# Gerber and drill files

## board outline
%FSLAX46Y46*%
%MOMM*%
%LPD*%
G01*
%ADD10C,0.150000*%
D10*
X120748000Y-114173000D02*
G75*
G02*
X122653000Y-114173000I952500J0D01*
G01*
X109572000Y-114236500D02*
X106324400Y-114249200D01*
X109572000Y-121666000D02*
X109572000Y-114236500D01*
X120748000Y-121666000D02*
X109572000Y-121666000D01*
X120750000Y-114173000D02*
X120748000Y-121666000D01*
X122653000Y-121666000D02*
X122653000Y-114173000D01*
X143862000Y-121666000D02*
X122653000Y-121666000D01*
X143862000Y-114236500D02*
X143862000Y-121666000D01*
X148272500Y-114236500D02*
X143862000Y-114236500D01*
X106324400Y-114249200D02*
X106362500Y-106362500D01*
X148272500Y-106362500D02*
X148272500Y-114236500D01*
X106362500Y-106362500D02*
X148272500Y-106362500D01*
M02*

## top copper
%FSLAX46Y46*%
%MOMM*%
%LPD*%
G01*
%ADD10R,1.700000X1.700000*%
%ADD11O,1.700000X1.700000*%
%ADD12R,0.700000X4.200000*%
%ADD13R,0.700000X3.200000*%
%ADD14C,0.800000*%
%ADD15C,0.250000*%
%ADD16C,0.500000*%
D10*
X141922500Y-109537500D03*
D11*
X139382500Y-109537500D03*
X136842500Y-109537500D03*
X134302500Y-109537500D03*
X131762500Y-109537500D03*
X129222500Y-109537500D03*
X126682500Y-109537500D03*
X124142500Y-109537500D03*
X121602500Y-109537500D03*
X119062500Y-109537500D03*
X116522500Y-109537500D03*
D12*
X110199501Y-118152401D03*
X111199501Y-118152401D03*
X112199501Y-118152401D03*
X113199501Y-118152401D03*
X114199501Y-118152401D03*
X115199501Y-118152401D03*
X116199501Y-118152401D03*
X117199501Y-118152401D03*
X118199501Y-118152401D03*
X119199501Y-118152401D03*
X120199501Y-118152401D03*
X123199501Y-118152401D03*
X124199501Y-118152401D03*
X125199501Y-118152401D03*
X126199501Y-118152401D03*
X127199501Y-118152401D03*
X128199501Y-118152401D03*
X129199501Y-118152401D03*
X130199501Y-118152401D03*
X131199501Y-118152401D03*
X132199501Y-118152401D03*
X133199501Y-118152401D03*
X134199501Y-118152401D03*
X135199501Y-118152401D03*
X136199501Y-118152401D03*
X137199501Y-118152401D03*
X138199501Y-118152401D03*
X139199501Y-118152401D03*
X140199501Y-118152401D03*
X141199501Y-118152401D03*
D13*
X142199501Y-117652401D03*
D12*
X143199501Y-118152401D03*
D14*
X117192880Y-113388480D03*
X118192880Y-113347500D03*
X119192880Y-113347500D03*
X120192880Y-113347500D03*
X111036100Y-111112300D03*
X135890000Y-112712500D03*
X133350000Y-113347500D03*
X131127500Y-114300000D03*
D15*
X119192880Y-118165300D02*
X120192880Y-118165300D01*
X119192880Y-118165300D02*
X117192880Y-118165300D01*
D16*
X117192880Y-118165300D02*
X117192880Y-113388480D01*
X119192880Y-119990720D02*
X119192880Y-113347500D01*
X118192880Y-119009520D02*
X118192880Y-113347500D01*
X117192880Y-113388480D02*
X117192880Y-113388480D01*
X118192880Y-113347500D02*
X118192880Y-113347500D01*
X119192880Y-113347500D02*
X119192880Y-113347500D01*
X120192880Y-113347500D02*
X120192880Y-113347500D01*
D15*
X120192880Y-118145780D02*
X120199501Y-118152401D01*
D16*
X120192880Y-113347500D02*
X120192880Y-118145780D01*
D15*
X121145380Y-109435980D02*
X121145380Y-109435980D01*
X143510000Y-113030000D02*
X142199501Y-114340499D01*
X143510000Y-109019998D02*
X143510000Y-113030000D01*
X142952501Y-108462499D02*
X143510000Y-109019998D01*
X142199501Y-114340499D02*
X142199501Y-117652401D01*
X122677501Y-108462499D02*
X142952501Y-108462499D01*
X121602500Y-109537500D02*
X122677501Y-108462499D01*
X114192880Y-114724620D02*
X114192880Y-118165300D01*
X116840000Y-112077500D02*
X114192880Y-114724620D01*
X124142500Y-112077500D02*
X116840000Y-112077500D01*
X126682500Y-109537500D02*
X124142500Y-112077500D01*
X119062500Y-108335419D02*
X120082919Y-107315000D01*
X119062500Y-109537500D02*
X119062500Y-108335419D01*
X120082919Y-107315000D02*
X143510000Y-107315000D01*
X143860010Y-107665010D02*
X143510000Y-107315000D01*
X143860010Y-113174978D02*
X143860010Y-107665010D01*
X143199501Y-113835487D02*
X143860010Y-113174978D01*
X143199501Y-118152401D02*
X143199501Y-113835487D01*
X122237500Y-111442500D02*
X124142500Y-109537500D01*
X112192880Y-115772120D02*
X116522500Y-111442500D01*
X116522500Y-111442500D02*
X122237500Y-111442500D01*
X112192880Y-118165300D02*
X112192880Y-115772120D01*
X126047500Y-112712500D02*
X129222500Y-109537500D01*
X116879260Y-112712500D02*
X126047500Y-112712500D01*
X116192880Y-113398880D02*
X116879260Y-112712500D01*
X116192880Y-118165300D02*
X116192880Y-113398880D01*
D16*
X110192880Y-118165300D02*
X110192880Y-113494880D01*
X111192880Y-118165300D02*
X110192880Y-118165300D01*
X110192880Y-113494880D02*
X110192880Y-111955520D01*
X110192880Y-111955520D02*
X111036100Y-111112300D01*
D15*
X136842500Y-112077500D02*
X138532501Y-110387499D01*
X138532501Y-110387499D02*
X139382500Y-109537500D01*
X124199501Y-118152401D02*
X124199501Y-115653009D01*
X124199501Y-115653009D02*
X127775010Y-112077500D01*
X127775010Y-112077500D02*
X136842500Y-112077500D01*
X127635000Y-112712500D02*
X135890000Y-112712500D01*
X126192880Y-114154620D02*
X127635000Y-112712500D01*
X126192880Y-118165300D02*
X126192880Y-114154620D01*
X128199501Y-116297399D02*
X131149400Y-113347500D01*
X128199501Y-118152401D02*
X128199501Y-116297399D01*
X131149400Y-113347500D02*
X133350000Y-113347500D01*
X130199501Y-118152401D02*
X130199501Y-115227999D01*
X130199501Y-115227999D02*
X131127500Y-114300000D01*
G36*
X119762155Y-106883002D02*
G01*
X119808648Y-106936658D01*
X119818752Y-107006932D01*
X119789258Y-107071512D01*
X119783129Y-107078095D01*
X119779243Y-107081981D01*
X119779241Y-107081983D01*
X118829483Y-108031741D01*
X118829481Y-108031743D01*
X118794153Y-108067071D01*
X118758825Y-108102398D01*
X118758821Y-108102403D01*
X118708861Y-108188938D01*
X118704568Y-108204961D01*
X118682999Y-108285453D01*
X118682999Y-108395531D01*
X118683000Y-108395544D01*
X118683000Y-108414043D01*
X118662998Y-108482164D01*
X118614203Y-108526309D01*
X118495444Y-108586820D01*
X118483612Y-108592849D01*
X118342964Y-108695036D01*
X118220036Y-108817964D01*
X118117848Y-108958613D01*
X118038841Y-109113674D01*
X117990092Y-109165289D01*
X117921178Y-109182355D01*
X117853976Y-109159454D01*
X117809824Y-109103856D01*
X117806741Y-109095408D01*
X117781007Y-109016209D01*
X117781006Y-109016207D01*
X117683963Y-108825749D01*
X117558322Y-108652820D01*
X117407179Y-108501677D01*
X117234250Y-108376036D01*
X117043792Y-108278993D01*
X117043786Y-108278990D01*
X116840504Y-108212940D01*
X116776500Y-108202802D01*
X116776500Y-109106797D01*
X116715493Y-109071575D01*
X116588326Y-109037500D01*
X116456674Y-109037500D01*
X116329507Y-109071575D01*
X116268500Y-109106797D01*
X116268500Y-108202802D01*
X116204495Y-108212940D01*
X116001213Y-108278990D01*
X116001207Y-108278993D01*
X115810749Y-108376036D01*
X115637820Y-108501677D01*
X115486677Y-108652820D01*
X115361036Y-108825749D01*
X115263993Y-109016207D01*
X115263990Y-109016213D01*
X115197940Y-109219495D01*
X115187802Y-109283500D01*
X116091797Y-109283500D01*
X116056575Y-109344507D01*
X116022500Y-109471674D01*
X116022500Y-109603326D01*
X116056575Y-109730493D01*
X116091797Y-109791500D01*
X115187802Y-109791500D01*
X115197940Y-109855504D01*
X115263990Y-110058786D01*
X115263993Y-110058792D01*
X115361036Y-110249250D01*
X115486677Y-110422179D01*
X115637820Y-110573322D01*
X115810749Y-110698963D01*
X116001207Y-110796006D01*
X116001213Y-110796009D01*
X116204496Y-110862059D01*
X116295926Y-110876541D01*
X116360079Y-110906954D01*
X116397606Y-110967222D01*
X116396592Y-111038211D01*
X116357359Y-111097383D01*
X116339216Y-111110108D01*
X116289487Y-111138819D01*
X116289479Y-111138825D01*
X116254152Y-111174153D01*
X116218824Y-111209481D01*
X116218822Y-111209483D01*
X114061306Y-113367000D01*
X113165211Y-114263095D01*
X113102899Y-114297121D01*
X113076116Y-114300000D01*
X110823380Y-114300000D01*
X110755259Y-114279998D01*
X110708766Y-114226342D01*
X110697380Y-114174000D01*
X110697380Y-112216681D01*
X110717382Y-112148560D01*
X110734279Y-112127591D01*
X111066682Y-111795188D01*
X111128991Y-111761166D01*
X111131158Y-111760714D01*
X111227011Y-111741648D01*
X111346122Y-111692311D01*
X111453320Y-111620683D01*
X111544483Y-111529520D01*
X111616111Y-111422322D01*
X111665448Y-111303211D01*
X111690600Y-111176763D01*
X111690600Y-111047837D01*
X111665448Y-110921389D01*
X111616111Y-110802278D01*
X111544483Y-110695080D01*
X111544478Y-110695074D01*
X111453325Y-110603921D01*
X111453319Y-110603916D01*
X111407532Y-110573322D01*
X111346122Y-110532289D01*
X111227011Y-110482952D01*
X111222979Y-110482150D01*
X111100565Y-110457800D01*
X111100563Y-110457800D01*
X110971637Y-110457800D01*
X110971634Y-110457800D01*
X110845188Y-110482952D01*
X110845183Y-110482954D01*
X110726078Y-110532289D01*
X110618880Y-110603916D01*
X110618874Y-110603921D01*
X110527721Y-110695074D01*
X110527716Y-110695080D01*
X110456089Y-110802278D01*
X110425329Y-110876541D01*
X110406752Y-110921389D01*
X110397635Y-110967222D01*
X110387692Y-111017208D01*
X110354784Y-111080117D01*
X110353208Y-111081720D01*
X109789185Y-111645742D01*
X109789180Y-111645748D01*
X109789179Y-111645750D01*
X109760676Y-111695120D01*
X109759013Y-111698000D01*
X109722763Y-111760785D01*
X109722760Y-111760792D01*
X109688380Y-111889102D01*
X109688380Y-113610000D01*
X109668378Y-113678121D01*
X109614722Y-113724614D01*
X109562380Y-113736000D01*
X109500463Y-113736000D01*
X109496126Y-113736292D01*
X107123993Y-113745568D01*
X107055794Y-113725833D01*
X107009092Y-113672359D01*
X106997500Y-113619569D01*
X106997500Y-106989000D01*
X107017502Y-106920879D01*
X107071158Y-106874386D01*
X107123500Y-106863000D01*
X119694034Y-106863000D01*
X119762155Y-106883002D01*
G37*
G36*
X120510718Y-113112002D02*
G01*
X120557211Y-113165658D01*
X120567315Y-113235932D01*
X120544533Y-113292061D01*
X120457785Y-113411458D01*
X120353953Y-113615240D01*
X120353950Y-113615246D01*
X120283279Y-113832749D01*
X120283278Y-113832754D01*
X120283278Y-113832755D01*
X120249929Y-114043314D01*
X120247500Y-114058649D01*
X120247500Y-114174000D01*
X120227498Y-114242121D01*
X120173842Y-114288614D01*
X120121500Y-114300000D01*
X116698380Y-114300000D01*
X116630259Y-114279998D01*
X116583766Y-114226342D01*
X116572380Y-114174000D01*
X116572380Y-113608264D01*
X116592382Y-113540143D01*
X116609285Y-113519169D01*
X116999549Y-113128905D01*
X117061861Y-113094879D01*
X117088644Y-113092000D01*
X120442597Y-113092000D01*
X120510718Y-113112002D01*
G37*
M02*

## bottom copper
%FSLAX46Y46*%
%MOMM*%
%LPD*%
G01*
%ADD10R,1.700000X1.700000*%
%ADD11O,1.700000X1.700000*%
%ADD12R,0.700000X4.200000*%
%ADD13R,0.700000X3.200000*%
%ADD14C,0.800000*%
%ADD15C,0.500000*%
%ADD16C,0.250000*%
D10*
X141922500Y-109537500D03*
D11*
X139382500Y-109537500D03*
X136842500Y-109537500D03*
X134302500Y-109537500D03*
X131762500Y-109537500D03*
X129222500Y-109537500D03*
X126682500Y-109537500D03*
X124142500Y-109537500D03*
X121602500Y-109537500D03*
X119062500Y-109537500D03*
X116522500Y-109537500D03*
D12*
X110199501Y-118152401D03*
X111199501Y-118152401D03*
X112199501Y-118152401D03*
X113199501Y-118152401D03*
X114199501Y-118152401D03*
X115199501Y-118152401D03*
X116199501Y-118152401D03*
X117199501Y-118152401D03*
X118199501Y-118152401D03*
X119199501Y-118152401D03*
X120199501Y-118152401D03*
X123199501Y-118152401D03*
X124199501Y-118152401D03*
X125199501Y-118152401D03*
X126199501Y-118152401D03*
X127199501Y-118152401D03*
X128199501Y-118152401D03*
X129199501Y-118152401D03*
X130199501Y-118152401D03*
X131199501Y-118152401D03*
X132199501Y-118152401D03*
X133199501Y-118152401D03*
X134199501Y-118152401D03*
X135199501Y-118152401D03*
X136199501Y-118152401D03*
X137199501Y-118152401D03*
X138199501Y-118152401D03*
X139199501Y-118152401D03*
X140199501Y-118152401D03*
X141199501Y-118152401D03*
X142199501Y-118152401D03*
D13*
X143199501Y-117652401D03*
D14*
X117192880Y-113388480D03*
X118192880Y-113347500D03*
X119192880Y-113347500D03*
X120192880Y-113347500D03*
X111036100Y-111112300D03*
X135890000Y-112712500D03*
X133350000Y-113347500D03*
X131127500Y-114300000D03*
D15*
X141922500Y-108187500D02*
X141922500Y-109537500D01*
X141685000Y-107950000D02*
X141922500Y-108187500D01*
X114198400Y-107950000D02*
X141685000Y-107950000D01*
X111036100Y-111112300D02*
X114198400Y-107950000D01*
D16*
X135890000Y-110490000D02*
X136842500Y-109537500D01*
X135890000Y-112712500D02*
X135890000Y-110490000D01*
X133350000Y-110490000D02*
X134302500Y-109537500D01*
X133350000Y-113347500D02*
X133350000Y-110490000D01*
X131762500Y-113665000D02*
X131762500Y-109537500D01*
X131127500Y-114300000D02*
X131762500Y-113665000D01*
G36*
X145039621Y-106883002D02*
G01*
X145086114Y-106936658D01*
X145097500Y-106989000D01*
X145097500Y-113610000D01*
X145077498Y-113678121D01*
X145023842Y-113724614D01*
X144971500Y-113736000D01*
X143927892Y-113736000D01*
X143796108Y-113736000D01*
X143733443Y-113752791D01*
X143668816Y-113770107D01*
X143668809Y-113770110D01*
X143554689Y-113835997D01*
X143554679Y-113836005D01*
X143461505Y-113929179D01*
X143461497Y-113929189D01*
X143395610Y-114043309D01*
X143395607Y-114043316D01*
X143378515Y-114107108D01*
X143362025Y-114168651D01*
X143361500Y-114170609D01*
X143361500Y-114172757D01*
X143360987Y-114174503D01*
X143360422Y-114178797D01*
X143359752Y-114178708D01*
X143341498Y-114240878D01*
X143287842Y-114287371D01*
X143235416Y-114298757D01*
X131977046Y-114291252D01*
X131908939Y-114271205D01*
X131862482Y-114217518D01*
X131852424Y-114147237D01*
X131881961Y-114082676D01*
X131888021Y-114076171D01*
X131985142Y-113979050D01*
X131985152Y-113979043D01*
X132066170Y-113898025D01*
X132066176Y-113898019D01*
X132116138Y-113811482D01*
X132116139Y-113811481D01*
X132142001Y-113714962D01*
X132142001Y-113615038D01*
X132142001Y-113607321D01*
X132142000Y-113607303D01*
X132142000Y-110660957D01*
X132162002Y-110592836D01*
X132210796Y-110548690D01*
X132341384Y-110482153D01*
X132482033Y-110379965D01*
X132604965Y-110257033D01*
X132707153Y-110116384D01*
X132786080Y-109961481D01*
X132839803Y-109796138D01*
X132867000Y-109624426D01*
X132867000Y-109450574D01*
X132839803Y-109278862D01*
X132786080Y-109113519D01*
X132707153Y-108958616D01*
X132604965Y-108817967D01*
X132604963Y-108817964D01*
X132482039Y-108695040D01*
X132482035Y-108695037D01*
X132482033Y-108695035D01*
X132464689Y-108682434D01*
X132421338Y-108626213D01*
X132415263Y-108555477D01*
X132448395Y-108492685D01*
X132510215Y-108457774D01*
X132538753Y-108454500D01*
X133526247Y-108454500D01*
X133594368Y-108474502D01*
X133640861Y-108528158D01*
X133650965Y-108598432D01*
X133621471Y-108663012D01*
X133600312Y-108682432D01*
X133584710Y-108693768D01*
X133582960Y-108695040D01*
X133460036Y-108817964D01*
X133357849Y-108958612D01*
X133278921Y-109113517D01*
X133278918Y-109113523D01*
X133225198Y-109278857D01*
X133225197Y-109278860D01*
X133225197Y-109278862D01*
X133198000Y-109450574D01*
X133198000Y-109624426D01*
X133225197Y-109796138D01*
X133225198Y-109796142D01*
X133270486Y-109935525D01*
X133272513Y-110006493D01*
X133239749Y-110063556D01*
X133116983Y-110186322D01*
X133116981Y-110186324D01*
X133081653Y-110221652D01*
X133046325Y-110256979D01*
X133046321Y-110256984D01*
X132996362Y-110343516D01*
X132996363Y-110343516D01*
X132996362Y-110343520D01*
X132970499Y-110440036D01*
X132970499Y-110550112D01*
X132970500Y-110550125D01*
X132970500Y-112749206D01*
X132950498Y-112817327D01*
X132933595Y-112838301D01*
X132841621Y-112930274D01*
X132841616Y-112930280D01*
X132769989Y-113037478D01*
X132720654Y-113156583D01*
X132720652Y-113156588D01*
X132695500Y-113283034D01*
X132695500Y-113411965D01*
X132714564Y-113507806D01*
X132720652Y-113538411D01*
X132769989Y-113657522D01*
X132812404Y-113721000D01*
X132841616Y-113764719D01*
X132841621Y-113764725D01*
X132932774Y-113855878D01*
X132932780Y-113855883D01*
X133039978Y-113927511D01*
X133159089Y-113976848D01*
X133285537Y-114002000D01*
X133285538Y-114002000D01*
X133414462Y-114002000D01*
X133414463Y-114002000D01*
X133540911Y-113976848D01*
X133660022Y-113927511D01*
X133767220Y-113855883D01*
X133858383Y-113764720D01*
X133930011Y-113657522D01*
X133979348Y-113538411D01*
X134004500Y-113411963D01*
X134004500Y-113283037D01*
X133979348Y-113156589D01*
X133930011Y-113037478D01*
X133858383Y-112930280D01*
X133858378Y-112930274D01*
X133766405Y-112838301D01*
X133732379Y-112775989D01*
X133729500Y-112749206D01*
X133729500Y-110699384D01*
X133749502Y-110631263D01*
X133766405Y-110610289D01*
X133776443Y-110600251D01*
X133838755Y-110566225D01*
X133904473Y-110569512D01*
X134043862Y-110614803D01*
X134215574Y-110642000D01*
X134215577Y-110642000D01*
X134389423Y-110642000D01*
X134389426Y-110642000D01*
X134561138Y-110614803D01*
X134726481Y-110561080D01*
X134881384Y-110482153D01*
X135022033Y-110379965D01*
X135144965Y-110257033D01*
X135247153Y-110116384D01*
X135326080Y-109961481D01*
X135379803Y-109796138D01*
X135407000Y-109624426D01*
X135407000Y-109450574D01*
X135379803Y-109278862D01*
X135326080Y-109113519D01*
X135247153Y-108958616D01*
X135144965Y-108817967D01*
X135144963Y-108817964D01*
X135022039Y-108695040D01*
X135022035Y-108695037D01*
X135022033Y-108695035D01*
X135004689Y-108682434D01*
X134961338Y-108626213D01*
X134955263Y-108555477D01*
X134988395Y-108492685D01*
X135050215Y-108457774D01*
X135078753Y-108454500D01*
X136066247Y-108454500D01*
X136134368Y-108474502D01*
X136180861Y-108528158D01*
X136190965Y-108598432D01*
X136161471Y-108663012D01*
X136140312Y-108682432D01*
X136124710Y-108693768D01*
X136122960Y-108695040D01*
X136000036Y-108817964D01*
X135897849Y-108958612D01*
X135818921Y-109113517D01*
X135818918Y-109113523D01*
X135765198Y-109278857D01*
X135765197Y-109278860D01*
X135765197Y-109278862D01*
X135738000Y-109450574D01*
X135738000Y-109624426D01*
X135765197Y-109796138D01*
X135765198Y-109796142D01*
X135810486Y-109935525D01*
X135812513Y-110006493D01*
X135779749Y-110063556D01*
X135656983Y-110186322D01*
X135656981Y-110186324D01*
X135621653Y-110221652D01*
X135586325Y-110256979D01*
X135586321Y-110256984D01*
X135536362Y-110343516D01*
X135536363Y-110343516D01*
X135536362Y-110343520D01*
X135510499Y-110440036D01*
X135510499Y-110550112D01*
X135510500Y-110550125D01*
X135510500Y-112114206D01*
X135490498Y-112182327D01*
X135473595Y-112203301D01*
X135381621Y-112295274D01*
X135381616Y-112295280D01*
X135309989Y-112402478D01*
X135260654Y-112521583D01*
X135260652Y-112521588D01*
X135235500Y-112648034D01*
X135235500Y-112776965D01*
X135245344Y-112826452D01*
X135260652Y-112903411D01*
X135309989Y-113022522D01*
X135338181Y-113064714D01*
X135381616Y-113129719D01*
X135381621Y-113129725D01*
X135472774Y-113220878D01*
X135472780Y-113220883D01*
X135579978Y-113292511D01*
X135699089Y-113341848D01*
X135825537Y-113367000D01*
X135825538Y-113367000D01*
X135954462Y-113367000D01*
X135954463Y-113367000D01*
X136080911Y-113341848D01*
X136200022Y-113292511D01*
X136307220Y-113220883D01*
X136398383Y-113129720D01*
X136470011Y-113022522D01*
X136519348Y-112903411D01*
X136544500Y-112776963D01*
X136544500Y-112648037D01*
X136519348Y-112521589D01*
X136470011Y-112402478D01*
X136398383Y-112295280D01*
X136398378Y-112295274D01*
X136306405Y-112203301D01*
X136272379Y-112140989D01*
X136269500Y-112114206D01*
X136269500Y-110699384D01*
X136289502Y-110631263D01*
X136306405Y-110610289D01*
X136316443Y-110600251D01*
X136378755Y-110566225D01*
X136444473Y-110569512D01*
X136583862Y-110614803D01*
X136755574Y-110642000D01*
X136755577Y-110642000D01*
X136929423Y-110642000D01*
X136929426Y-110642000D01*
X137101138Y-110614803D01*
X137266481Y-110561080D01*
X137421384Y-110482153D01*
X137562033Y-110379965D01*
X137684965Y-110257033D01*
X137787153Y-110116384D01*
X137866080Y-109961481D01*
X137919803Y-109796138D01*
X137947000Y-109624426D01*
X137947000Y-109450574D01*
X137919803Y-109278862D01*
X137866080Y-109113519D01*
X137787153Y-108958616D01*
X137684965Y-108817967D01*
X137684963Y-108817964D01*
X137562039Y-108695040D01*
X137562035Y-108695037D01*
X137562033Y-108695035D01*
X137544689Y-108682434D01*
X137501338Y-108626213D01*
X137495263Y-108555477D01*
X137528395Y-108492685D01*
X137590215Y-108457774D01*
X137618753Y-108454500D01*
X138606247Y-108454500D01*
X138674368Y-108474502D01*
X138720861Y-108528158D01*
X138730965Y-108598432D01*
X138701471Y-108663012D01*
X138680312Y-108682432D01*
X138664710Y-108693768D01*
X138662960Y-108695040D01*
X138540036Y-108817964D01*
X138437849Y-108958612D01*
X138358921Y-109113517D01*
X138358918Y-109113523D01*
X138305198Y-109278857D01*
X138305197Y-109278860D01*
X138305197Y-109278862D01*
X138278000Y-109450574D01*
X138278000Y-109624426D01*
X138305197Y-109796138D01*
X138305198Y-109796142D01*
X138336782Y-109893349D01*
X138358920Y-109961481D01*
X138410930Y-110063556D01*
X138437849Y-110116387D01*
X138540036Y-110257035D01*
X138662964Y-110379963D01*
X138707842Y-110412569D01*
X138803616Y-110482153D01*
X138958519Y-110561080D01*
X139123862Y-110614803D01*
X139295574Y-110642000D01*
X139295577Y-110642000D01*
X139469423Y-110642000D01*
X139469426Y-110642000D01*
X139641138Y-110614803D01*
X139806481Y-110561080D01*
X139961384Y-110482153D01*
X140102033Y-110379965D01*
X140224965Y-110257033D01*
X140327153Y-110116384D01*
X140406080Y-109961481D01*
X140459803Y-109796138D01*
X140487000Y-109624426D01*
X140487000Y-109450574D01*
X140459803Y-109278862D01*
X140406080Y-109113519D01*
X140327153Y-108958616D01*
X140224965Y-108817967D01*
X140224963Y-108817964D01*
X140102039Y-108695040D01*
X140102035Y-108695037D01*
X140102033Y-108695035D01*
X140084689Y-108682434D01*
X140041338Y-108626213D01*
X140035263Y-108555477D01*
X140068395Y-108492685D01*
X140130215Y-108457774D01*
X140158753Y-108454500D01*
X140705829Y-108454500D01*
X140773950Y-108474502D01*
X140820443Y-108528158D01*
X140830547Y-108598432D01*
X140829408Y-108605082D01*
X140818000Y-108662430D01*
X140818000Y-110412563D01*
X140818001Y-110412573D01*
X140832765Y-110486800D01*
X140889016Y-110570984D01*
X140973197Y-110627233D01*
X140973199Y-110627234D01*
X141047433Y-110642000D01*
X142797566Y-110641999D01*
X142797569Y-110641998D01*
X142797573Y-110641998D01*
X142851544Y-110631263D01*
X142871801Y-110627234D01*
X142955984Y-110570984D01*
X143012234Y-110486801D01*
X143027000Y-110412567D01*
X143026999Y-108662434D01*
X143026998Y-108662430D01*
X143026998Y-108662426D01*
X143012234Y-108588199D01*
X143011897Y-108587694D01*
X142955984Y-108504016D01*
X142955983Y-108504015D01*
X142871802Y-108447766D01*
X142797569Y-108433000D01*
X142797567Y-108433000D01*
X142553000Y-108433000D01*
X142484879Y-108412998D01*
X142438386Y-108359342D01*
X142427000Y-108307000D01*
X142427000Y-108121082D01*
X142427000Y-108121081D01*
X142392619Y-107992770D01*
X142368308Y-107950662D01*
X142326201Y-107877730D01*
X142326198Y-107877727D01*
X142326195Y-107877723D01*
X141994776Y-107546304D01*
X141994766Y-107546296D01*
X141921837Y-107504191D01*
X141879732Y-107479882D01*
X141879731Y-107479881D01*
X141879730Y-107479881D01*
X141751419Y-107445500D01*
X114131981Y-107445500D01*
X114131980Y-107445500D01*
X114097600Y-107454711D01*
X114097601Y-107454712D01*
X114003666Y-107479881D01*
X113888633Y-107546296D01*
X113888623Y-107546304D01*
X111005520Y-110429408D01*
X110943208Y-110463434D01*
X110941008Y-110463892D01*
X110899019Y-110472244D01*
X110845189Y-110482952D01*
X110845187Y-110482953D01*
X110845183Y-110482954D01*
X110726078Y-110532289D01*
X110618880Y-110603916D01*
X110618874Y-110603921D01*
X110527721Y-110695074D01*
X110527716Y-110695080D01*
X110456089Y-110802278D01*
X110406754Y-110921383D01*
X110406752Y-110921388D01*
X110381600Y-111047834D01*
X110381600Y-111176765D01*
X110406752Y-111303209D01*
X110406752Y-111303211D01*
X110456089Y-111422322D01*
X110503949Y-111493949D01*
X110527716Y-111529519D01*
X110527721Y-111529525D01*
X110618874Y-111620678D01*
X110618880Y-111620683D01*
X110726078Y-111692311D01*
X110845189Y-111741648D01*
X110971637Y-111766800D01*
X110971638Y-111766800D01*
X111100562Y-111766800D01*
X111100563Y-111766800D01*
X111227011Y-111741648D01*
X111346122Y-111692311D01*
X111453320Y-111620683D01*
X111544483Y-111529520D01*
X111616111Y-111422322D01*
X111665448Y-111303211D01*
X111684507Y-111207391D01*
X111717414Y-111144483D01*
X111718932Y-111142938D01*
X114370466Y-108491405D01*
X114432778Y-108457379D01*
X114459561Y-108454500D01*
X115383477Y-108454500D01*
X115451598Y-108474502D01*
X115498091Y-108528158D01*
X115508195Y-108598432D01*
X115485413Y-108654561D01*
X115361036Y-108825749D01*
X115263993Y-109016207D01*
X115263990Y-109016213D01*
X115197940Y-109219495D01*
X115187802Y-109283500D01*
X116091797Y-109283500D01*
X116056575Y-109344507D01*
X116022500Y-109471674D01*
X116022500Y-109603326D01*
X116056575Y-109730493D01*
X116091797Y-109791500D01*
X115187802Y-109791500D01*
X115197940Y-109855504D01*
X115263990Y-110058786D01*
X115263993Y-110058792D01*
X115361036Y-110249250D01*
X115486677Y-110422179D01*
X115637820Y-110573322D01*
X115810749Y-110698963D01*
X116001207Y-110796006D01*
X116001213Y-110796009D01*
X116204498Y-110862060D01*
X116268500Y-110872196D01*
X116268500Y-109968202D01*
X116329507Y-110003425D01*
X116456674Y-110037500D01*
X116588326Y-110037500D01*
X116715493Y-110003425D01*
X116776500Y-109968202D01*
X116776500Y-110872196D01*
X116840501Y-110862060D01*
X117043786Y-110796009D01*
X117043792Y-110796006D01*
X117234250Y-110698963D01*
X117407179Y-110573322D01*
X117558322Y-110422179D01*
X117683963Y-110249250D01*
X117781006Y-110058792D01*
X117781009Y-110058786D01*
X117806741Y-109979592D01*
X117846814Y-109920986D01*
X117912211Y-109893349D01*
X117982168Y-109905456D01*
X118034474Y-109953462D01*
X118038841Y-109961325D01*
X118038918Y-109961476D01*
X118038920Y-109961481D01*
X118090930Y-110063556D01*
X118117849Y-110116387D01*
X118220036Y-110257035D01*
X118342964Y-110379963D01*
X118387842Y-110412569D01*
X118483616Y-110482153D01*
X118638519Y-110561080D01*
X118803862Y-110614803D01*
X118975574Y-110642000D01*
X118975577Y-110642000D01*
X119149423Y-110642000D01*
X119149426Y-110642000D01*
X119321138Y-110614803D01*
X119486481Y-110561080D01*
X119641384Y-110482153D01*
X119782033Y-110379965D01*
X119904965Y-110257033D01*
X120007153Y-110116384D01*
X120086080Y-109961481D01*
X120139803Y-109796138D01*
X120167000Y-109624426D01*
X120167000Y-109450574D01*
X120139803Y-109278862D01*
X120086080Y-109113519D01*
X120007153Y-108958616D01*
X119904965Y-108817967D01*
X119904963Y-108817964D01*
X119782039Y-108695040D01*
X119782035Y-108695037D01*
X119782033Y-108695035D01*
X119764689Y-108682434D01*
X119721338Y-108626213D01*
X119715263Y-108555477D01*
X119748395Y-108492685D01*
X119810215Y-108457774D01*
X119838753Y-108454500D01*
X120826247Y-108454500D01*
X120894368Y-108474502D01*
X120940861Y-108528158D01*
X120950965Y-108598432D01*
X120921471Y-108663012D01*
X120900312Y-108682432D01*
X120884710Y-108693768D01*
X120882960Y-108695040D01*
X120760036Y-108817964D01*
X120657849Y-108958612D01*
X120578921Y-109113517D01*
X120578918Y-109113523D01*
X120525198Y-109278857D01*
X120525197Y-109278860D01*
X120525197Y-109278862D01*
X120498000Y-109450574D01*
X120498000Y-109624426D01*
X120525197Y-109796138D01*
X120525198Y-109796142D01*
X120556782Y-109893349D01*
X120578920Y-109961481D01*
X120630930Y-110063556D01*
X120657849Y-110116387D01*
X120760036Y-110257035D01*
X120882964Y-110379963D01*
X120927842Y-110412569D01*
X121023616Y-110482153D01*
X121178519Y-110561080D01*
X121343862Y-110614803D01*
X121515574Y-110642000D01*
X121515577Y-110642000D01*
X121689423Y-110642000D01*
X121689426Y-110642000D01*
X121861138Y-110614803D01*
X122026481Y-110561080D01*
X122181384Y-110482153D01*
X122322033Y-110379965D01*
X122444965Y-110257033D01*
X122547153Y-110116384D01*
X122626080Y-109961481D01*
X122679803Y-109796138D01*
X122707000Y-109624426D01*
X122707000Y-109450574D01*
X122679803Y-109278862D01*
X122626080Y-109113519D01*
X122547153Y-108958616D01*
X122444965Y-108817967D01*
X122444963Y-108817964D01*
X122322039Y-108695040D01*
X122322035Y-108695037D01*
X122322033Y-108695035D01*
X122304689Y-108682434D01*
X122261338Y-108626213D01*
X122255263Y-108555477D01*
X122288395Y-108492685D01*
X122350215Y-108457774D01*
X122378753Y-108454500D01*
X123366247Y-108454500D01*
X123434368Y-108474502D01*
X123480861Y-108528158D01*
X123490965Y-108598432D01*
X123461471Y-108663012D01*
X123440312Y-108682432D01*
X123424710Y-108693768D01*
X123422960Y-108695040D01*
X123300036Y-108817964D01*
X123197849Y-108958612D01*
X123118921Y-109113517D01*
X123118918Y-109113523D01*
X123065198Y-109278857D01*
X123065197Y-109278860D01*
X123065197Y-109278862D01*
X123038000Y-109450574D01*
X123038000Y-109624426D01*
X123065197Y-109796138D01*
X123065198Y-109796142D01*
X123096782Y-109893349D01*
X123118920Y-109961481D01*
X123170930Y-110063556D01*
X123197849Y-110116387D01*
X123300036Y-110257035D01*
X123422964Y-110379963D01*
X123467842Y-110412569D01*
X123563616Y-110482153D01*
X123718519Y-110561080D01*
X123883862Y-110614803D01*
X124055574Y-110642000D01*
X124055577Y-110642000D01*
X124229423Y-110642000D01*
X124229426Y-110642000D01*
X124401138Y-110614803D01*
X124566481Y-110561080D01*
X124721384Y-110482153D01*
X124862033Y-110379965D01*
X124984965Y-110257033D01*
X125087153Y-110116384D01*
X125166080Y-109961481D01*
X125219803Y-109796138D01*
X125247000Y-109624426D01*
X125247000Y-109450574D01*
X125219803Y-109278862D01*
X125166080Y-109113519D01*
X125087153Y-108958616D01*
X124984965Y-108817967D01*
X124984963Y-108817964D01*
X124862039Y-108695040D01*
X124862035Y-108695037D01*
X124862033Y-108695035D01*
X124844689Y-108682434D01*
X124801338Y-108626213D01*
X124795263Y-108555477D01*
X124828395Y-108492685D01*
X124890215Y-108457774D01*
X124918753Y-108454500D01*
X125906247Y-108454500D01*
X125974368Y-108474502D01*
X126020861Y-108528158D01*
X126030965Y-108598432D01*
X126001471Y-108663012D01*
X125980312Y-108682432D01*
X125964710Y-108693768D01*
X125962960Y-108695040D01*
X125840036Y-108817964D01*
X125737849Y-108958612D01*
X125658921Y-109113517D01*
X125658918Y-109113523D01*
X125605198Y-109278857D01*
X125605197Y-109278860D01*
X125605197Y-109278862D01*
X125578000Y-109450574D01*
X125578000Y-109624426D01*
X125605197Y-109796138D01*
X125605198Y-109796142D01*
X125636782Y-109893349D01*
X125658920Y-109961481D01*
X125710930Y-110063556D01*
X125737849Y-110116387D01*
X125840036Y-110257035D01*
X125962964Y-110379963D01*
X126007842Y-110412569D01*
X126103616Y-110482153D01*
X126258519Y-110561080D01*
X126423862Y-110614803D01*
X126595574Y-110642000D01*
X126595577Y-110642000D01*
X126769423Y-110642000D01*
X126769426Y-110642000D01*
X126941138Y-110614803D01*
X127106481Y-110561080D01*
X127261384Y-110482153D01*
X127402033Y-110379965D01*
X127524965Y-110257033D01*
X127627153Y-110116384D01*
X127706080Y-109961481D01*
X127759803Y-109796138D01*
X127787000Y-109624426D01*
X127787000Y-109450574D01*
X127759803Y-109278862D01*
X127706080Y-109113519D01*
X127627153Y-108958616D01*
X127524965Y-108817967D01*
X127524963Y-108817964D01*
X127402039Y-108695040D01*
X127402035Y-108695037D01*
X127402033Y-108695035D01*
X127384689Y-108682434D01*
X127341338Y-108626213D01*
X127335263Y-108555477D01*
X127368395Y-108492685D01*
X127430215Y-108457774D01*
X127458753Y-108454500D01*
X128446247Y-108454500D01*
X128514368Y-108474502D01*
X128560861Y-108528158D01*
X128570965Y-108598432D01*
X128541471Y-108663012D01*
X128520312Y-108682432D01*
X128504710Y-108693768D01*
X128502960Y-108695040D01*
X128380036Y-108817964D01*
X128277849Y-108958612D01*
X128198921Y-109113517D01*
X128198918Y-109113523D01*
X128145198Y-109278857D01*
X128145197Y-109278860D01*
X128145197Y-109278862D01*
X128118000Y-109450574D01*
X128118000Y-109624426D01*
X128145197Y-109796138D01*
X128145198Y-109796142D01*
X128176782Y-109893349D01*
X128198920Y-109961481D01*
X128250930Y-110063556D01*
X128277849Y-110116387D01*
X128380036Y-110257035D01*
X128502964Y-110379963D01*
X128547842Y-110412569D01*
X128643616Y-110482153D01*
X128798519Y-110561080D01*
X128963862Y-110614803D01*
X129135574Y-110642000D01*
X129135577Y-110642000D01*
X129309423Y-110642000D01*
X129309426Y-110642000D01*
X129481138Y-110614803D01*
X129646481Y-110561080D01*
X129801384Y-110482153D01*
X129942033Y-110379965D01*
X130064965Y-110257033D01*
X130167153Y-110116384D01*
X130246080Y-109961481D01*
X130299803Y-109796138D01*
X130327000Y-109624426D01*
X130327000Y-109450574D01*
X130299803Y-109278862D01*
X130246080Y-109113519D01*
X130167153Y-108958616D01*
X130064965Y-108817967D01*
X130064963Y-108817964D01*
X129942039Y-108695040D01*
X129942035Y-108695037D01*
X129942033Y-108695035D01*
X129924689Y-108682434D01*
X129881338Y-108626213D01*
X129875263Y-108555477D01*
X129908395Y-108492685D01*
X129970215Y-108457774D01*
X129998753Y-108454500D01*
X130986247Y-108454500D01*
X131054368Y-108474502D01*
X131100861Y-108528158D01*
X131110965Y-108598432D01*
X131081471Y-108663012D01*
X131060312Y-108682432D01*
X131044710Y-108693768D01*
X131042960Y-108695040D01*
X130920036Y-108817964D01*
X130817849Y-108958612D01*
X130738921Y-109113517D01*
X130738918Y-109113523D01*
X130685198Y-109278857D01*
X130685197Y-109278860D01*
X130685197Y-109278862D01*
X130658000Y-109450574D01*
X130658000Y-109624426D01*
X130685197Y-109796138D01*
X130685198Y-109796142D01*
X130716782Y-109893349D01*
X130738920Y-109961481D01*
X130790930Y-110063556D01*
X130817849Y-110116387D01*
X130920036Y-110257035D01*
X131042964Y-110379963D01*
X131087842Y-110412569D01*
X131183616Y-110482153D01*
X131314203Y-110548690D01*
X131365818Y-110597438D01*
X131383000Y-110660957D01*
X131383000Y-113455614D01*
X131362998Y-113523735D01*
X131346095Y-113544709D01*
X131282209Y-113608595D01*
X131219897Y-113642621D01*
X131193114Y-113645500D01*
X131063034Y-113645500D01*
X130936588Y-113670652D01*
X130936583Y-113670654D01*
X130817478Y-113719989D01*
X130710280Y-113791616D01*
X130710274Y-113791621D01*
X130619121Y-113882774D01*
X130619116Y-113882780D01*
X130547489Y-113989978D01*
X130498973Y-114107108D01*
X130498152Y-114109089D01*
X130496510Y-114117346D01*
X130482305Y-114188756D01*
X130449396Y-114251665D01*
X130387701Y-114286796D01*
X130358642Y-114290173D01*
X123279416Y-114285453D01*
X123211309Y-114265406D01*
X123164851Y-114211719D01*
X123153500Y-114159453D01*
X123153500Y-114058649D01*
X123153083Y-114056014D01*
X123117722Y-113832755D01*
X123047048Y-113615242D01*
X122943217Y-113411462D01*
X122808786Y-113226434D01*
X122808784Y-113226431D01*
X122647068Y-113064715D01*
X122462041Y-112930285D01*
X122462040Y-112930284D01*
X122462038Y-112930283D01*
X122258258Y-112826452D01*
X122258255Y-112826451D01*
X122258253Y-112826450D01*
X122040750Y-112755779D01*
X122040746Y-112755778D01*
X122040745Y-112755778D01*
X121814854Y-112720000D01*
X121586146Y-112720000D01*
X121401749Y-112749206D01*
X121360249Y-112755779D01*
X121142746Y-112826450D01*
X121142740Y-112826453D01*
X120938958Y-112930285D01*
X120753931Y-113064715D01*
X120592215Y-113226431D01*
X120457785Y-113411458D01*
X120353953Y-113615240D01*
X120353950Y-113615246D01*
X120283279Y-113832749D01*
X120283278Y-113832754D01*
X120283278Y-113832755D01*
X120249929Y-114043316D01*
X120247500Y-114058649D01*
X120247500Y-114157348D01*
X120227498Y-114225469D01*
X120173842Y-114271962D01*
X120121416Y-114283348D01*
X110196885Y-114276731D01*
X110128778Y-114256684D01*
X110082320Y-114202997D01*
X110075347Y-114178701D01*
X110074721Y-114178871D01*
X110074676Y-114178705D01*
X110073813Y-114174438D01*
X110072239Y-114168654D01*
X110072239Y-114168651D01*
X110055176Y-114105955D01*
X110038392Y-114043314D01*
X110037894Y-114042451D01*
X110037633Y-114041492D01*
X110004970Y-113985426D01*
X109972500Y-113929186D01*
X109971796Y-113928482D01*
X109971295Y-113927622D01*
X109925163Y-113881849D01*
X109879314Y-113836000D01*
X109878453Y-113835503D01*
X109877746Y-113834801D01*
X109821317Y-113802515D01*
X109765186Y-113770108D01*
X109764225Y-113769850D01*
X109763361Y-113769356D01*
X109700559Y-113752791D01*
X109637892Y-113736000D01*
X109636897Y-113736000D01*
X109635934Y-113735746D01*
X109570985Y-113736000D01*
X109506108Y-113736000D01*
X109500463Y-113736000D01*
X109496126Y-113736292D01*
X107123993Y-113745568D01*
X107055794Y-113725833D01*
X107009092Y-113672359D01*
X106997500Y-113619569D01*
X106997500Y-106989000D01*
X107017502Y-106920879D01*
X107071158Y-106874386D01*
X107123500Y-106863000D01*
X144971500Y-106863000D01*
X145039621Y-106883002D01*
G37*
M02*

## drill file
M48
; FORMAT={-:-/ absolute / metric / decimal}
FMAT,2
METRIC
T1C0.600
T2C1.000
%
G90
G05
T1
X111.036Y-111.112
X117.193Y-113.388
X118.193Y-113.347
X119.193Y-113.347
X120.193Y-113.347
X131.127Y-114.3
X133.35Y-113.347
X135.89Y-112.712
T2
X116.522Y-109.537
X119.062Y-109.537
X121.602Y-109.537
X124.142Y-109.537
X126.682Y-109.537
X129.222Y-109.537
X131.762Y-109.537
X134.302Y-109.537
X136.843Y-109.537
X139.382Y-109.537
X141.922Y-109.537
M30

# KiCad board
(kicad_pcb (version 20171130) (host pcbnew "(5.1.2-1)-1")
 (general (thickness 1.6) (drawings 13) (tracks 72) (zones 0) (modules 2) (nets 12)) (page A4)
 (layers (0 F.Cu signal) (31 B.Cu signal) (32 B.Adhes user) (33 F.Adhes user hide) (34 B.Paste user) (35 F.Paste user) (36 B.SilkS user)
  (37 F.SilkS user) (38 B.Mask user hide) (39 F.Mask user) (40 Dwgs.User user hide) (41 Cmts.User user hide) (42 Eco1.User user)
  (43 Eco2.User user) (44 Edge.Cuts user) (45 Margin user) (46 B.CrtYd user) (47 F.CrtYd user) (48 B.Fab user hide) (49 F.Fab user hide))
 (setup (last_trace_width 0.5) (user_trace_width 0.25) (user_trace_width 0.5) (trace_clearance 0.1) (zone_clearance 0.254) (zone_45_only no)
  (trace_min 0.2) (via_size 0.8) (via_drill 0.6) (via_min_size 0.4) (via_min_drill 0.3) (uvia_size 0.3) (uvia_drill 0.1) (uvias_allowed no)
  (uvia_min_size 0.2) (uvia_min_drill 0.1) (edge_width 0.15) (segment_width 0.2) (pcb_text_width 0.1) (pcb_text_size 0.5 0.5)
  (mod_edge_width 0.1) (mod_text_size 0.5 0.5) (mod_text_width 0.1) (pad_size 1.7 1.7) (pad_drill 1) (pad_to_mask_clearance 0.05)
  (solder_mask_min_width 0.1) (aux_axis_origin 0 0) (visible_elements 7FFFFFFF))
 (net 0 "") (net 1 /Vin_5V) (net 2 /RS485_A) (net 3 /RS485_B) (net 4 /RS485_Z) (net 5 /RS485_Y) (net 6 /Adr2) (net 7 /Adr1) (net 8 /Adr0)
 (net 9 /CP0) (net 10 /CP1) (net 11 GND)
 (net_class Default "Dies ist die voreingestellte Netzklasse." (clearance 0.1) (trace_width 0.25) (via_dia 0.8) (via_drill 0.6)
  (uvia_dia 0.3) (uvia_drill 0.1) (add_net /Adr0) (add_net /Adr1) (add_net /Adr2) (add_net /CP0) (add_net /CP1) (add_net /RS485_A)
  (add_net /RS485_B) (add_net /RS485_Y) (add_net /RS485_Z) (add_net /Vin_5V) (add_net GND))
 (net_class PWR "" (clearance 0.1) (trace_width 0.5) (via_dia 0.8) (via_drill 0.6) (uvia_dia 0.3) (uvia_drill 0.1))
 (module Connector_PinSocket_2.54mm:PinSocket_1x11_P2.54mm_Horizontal (layer F.Cu) (at 141.9225 109.5375 270)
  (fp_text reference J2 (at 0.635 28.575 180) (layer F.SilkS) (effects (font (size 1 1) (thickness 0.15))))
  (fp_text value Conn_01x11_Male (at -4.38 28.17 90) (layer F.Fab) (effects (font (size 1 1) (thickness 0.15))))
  (pad 1 thru_hole rect (at 0 0 270) (size 1.7 1.7) (drill 1) (layers *.Cu *.Mask) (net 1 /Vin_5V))
  (pad 2 thru_hole oval (at 0 2.54 270) (size 1.7 1.7) (drill 1) (layers *.Cu *.Mask) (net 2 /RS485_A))
  (pad 3 thru_hole oval (at 0 5.08 270) (size 1.7 1.7) (drill 1) (layers *.Cu *.Mask) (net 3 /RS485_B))
  (pad 4 thru_hole oval (at 0 7.62 270) (size 1.7 1.7) (drill 1) (layers *.Cu *.Mask) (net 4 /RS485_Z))
  (pad 5 thru_hole oval (at 0 10.16 270) (size 1.7 1.7) (drill 1) (layers *.Cu *.Mask) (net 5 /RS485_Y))
  (pad 6 thru_hole oval (at 0 12.7 270) (size 1.7 1.7) (drill 1) (layers *.Cu *.Mask) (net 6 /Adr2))
  (pad 7 thru_hole oval (at 0 15.24 270) (size 1.7 1.7) (drill 1) (layers *.Cu *.Mask) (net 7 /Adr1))
  (pad 8 thru_hole oval (at 0 17.78 270) (size 1.7 1.7) (drill 1) (layers *.Cu *.Mask) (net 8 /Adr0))
  (pad 9 thru_hole oval (at 0 20.32 270) (size 1.7 1.7) (drill 1) (layers *.Cu *.Mask) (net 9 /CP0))
  (pad 10 thru_hole oval (at 0 22.86 270) (size 1.7 1.7) (drill 1) (layers *.Cu *.Mask) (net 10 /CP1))
  (pad 11 thru_hole oval (at 0 25.4 270) (size 1.7 1.7) (drill 1) (layers *.Cu *.Mask) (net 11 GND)))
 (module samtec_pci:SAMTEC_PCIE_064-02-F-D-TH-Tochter (layer F.Cu) (at 121.699501 116.052401)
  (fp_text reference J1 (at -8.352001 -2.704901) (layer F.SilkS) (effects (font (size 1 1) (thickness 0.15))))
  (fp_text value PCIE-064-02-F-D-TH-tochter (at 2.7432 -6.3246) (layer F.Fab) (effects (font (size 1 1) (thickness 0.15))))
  (pad B1 connect rect (at -11.5 2.1) (size 0.7 4.2) (layers F.Cu F.Mask) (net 1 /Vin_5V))
  (pad B2 connect rect (at -10.5 2.1) (size 0.7 4.2) (layers F.Cu F.Mask) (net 1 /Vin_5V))
  (pad B3 connect rect (at -9.5 2.1) (size 0.7 4.2) (layers F.Cu F.Mask) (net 8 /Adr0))
  (pad B4 connect rect (at -8.5 2.1) (size 0.7 4.2) (layers F.Cu F.Mask))
  (pad B5 connect rect (at -7.5 2.1) (size 0.7 4.2) (layers F.Cu F.Mask) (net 7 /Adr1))
  (pad B6 connect rect (at -6.5 2.1) (size 0.7 4.2) (layers F.Cu F.Mask))
  (pad B7 connect rect (at -5.5 2.1) (size 0.7 4.2) (layers F.Cu F.Mask) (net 6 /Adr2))
  (pad B8 connect rect (at -4.5 2.1) (size 0.7 4.2) (layers F.Cu F.Mask) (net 11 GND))
  (pad B9 connect rect (at -3.5 2.1) (size 0.7 4.2) (layers F.Cu F.Mask) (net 11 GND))
  (pad B10 connect rect (at -2.5 2.1) (size 0.7 4.2) (layers F.Cu F.Mask) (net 11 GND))
  (pad B11 connect rect (at -1.5 2.1) (size 0.7 4.2) (layers F.Cu F.Mask) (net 11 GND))
  (pad B12 connect rect (at 1.5 2.1) (size 0.7 4.2) (layers F.Cu F.Mask))
  (pad B13 connect rect (at 2.5 2.1) (size 0.7 4.2) (layers F.Cu F.Mask) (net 2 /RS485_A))
  (pad B14 connect rect (at 3.5 2.1) (size 0.7 4.2) (layers F.Cu F.Mask))
  (pad B15 connect rect (at 4.5 2.1) (size 0.7 4.2) (layers F.Cu F.Mask) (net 3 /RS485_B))
  (pad B16 connect rect (at 5.5 2.1) (size 0.7 4.2) (layers F.Cu F.Mask))
  (pad B17 connect rect (at 6.5 2.1) (size 0.7 4.2) (layers F.Cu F.Mask) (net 4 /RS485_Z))
  (pad B18 connect rect (at 7.5 2.1) (size 0.7 4.2) (layers F.Cu F.Mask))
  (pad B19 connect rect (at 8.5 2.1) (size 0.7 4.2) (layers F.Cu F.Mask) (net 5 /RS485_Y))
  (pad B20 connect rect (at 9.5 2.1) (size 0.7 4.2) (layers F.Cu F.Mask))
  (pad B21 connect rect (at 10.5 2.1) (size 0.7 4.2) (layers F.Cu F.Mask))
  (pad B22 connect rect (at 11.5 2.1) (size 0.7 4.2) (layers F.Cu F.Mask))
  (pad B23 connect rect (at 12.5 2.1) (size 0.7 4.2) (layers F.Cu F.Mask))
  (pad B24 connect rect (at 13.5 2.1) (size 0.7 4.2) (layers F.Cu F.Mask))
  (pad B25 connect rect (at 14.5 2.1) (size 0.7 4.2) (layers F.Cu F.Mask))
  (pad B26 connect rect (at 15.5 2.1) (size 0.7 4.2) (layers F.Cu F.Mask))
  (pad B27 connect rect (at 16.5 2.1) (size 0.7 4.2) (layers F.Cu F.Mask))
  (pad B28 connect rect (at 17.5 2.1) (size 0.7 4.2) (layers F.Cu F.Mask))
  (pad B29 connect rect (at 18.5 2.1) (size 0.7 4.2) (layers F.Cu F.Mask))
  (pad B30 connect rect (at 19.5 2.1) (size 0.7 4.2) (layers F.Cu F.Mask))
  (pad B31 connect rect (at 20.5 1.6) (size 0.7 3.2) (layers F.Cu F.Mask) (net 9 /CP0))
  (pad B32 connect rect (at 21.5 2.1) (size 0.7 4.2) (layers F.Cu F.Mask) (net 10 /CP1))
  (pad A1 connect rect (at -11.5 2.1) (size 0.7 4.2) (layers B.Cu F.Mask))
  (pad A2 connect rect (at -10.5 2.1) (size 0.7 4.2) (layers B.Cu F.Mask))
  (pad A3 connect rect (at -9.5 2.1) (size 0.7 4.2) (layers B.Cu F.Mask))
  (pad A4 connect rect (at -8.5 2.1) (size 0.7 4.2) (layers B.Cu F.Mask))
  (pad A5 connect rect (at -7.5 2.1) (size 0.7 4.2) (layers B.Cu F.Mask))
  (pad A6 connect rect (at -6.5 2.1) (size 0.7 4.2) (layers B.Cu F.Mask))
  (pad A7 connect rect (at -5.5 2.1) (size 0.7 4.2) (layers B.Cu F.Mask))
  (pad A8 connect rect (at -4.5 2.1) (size 0.7 4.2) (layers B.Cu F.Mask))
  (pad A9 connect rect (at -3.5 2.1) (size 0.7 4.2) (layers B.Cu F.Mask))
  (pad A10 connect rect (at -2.5 2.1) (size 0.7 4.2) (layers B.Cu F.Mask))
  (pad A11 connect rect (at -1.5 2.1) (size 0.7 4.2) (layers B.Cu F.Mask))
  (pad A12 connect rect (at 1.5 2.1) (size 0.7 4.2) (layers B.Cu F.Mask))
  (pad A13 connect rect (at 2.5 2.1) (size 0.7 4.2) (layers B.Cu F.Mask))
  (pad A14 connect rect (at 3.5 2.1) (size 0.7 4.2) (layers B.Cu F.Mask))
  (pad A15 connect rect (at 4.5 2.1) (size 0.7 4.2) (layers B.Cu F.Mask))
  (pad A16 connect rect (at 5.5 2.1) (size 0.7 4.2) (layers B.Cu F.Mask))
  (pad A17 connect rect (at 6.5 2.1) (size 0.7 4.2) (layers B.Cu F.Mask))
  (pad A18 connect rect (at 7.5 2.1) (size 0.7 4.2) (layers B.Cu F.Mask))
  (pad A19 connect rect (at 8.5 2.1) (size 0.7 4.2) (layers B.Cu F.Mask))
  (pad A20 connect rect (at 9.5 2.1) (size 0.7 4.2) (layers B.Cu F.Mask))
  (pad A21 connect rect (at 10.5 2.1) (size 0.7 4.2) (layers B.Cu F.Mask))
  (pad A22 connect rect (at 11.5 2.1) (size 0.7 4.2) (layers B.Cu F.Mask))
  (pad A23 connect rect (at 12.5 2.1) (size 0.7 4.2) (layers B.Cu F.Mask))
  (pad A24 connect rect (at 13.5 2.1) (size 0.7 4.2) (layers B.Cu F.Mask))
  (pad A25 connect rect (at 14.5 2.1) (size 0.7 4.2) (layers B.Cu F.Mask))
  (pad A26 connect rect (at 15.5 2.1) (size 0.7 4.2) (layers B.Cu F.Mask))
  (pad A27 connect rect (at 16.5 2.1) (size 0.7 4.2) (layers B.Cu F.Mask))
  (pad A28 connect rect (at 17.5 2.1) (size 0.7 4.2) (layers B.Cu F.Mask))
  (pad A29 connect rect (at 18.5 2.1) (size 0.7 4.2) (layers B.Cu F.Mask))
  (pad A30 connect rect (at 19.5 2.1) (size 0.7 4.2) (layers B.Cu F.Mask))
  (pad A31 connect rect (at 20.5 2.1) (size 0.7 4.2) (layers B.Cu F.Mask))
  (pad A32 connect rect (at 21.5 1.6) (size 0.7 3.2) (layers B.Cu F.Mask)))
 (gr_arc (start 121.7005 114.173) (end 122.653 114.173) (angle -180) (layer Edge.Cuts) (width 0.15))
 (gr_line (start 109.572 114.2365) (end 106.3244 114.2492) (layer Edge.Cuts) (width 0.15))
 (gr_line (start 109.572 121.666) (end 109.572 114.2365) (layer Edge.Cuts) (width 0.15))
 (gr_line (start 120.748 121.666) (end 109.572 121.666) (layer Edge.Cuts) (width 0.15))
 (gr_line (start 120.75 114.173) (end 120.748 121.666) (layer Edge.Cuts) (width 0.15))
 (gr_line (start 122.653 121.666) (end 122.653 114.173) (layer Edge.Cuts) (width 0.15))
 (gr_line (start 143.862 121.666) (end 122.653 121.666) (layer Edge.Cuts) (width 0.15))
 (gr_line (start 143.862 114.2365) (end 143.862 121.666) (layer Edge.Cuts) (width 0.15))
 (gr_line (start 148.2725 114.2365) (end 143.862 114.2365) (layer Edge.Cuts) (width 0.15))
 (gr_line (start 106.3244 114.2492) (end 106.3625 106.3625) (layer Edge.Cuts) (width 0.15))
 (gr_line (start 148.2725 106.3625) (end 148.2725 114.2365) (layer Edge.Cuts) (width 0.15))
 (gr_line (start 106.3625 106.3625) (end 148.2725 106.3625) (layer Edge.Cuts) (width 0.15))
 (segment (start 119.19288 118.1653) (end 120.19288 118.1653) (width 0.25) (layer F.Cu) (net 11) (status 30))
 (segment (start 119.19288 118.1653) (end 117.19288 118.1653) (width 0.25) (layer F.Cu) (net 11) (status 30))
 (segment (start 117.19288 118.1653) (end 117.19288 113.38848) (width 0.5) (layer F.Cu) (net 11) (status 10))
 (segment (start 119.19288 119.99072) (end 119.19288 113.3475) (width 0.5) (layer F.Cu) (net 11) (status 10))
 (segment (start 118.19288 119.00952) (end 118.19288 113.3475) (width 0.5) (layer F.Cu) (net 11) (status 10))
 (segment (start 117.19288 113.38848) (end 117.19288 113.38848) (width 0.5) (layer F.Cu) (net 11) (status 10))
 (via (at 117.19288 113.38848) (size 0.8) (drill 0.6) (layers F.Cu B.Cu) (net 11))
 (segment (start 118.19288 113.3475) (end 118.19288 113.3475) (width 0.5) (layer F.Cu) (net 11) (status 10))
 (via (at 118.19288 113.3475) (size 0.8) (drill 0.6) (layers F.Cu B.Cu) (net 11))
 (segment (start 119.19288 113.3475) (end 119.19288 113.3475) (width 0.5) (layer F.Cu) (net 11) (status 10))
 (via (at 119.19288 113.3475) (size 0.8) (drill 0.6) (layers F.Cu B.Cu) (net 11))
 (segment (start 120.19288 113.3475) (end 120.19288 113.3475) (width 0.5) (layer F.Cu) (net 11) (status 10))
 (via (at 120.19288 113.3475) (size 0.8) (drill 0.6) (layers F.Cu B.Cu) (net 11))
 (segment (start 120.19288 118.14578) (end 120.199501 118.152401) (width 0.25) (layer F.Cu) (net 11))
 (segment (start 120.19288 113.3475) (end 120.19288 118.14578) (width 0.5) (layer F.Cu) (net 11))
 (segment (start 121.14538 109.43598) (end 121.14538 109.43598) (width 0.25) (layer F.Cu) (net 9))
 (segment (start 143.51 113.03) (end 142.199501 114.340499) (width 0.25) (layer F.Cu) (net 9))
 (segment (start 143.51 109.019998) (end 143.51 113.03) (width 0.25) (layer F.Cu) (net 9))
 (segment (start 142.952501 108.462499) (end 143.51 109.019998) (width 0.25) (layer F.Cu) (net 9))
 (segment (start 142.199501 114.340499) (end 142.199501 117.652401) (width 0.25) (layer F.Cu) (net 9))
 (segment (start 122.677501 108.462499) (end 142.952501 108.462499) (width 0.25) (layer F.Cu) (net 9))
 (segment (start 121.6025 109.5375) (end 122.677501 108.462499) (width 0.25) (layer F.Cu) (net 9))
 (segment (start 114.19288 114.72462) (end 114.19288 118.1653) (width 0.25) (layer F.Cu) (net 7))
 (segment (start 116.84 112.0775) (end 114.19288 114.72462) (width 0.25) (layer F.Cu) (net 7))
 (segment (start 124.1425 112.0775) (end 116.84 112.0775) (width 0.25) (layer F.Cu) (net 7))
 (segment (start 126.6825 109.5375) (end 124.1425 112.0775) (width 0.25) (layer F.Cu) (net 7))
 (segment (start 119.0625 108.335419) (end 120.082919 107.315) (width 0.25) (layer F.Cu) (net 10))
 (segment (start 119.0625 109.5375) (end 119.0625 108.335419) (width 0.25) (layer F.Cu) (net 10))
 (segment (start 120.082919 107.315) (end 143.51 107.315) (width 0.25) (layer F.Cu) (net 10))
 (segment (start 143.86001 107.66501) (end 143.51 107.315) (width 0.25) (layer F.Cu) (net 10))
 (segment (start 143.86001 113.174978) (end 143.86001 107.66501) (width 0.25) (layer F.Cu) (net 10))
 (segment (start 143.199501 113.835487) (end 143.86001 113.174978) (width 0.25) (layer F.Cu) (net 10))
 (segment (start 143.199501 118.152401) (end 143.199501 113.835487) (width 0.25) (layer F.Cu) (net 10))
 (segment (start 122.2375 111.4425) (end 124.1425 109.5375) (width 0.25) (layer F.Cu) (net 8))
 (segment (start 112.19288 115.77212) (end 116.5225 111.4425) (width 0.25) (layer F.Cu) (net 8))
 (segment (start 116.5225 111.4425) (end 122.2375 111.4425) (width 0.25) (layer F.Cu) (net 8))
 (segment (start 112.19288 118.1653) (end 112.19288 115.77212) (width 0.25) (layer F.Cu) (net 8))
 (segment (start 126.0475 112.7125) (end 129.2225 109.5375) (width 0.25) (layer F.Cu) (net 6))
 (segment (start 116.87926 112.7125) (end 126.0475 112.7125) (width 0.25) (layer F.Cu) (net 6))
 (segment (start 116.19288 113.39888) (end 116.87926 112.7125) (width 0.25) (layer F.Cu) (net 6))
 (segment (start 116.19288 118.1653) (end 116.19288 113.39888) (width 0.25) (layer F.Cu) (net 6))
 (segment (start 110.19288 118.1653) (end 110.19288 113.49488) (width 0.5) (layer F.Cu) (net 1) (status 10))
 (segment (start 111.19288 118.1653) (end 110.19288 118.1653) (width 0.5) (layer F.Cu) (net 1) (status 30))
 (segment (start 110.19288 113.49488) (end 110.19288 111.95552) (width 0.5) (layer F.Cu) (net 1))
 (segment (start 110.19288 111.95552) (end 111.0361 111.1123) (width 0.5) (layer F.Cu) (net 1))
 (via (at 111.0361 111.1123) (size 0.8) (drill 0.6) (layers F.Cu B.Cu) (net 1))
 (segment (start 141.9225 108.1875) (end 141.9225 109.5375) (width 0.5) (layer B.Cu) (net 1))
 (segment (start 141.685 107.95) (end 141.9225 108.1875) (width 0.5) (layer B.Cu) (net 1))
 (segment (start 114.1984 107.95) (end 141.685 107.95) (width 0.5) (layer B.Cu) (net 1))
 (segment (start 111.0361 111.1123) (end 114.1984 107.95) (width 0.5) (layer B.Cu) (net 1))
 (segment (start 136.8425 112.0775) (end 138.532501 110.387499) (width 0.25) (layer F.Cu) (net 2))
 (segment (start 138.532501 110.387499) (end 139.3825 109.5375) (width 0.25) (layer F.Cu) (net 2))
 (segment (start 124.199501 118.152401) (end 124.199501 115.653009) (width 0.25) (layer F.Cu) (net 2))
 (segment (start 124.199501 115.653009) (end 127.77501 112.0775) (width 0.25) (layer F.Cu) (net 2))
 (segment (start 127.77501 112.0775) (end 136.8425 112.0775) (width 0.25) (layer F.Cu) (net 2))
 (via (at 135.89 112.7125) (size 0.8) (drill 0.6) (layers F.Cu B.Cu) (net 3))
 (segment (start 135.89 110.49) (end 136.8425 109.5375) (width 0.25) (layer B.Cu) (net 3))
 (segment (start 135.89 112.7125) (end 135.89 110.49) (width 0.25) (layer B.Cu) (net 3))
 (segment (start 127.635 112.7125) (end 135.89 112.7125) (width 0.25) (layer F.Cu) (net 3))
 (segment (start 126.19288 114.15462) (end 127.635 112.7125) (width 0.25) (layer F.Cu) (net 3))
 (segment (start 126.19288 118.1653) (end 126.19288 114.15462) (width 0.25) (layer F.Cu) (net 3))
 (segment (start 128.199501 116.297399) (end 131.1494 113.3475) (width 0.25) (layer F.Cu) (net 4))
 (segment (start 128.199501 118.152401) (end 128.199501 116.297399) (width 0.25) (layer F.Cu) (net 4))
 (segment (start 131.1494 113.3475) (end 133.35 113.3475) (width 0.25) (layer F.Cu) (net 4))
 (via (at 133.35 113.3475) (size 0.8) (drill 0.6) (layers F.Cu B.Cu) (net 4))
 (segment (start 133.35 110.49) (end 134.3025 109.5375) (width 0.25) (layer B.Cu) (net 4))
 (segment (start 133.35 113.3475) (end 133.35 110.49) (width 0.25) (layer B.Cu) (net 4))
 (segment (start 130.199501 118.152401) (end 130.199501 115.227999) (width 0.25) (layer F.Cu) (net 5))
 (segment (start 130.199501 115.227999) (end 131.1275 114.3) (width 0.25) (layer F.Cu) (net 5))
 (via (at 131.1275 114.3) (size 0.8) (drill 0.6) (layers F.Cu B.Cu) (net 5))
 (segment (start 131.7625 113.665) (end 131.7625 109.5375) (width 0.25) (layer B.Cu) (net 5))
 (segment (start 131.1275 114.3) (end 131.7625 113.665) (width 0.25) (layer B.Cu) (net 5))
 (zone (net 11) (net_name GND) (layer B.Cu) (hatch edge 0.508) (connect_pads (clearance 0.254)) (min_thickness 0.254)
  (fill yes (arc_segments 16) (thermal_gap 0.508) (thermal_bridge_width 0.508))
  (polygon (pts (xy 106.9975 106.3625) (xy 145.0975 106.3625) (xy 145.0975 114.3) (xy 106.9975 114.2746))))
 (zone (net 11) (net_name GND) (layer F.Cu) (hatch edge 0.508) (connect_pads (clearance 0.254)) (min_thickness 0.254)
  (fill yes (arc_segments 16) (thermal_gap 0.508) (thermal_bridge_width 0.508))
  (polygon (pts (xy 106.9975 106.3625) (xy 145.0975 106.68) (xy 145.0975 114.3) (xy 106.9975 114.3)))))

